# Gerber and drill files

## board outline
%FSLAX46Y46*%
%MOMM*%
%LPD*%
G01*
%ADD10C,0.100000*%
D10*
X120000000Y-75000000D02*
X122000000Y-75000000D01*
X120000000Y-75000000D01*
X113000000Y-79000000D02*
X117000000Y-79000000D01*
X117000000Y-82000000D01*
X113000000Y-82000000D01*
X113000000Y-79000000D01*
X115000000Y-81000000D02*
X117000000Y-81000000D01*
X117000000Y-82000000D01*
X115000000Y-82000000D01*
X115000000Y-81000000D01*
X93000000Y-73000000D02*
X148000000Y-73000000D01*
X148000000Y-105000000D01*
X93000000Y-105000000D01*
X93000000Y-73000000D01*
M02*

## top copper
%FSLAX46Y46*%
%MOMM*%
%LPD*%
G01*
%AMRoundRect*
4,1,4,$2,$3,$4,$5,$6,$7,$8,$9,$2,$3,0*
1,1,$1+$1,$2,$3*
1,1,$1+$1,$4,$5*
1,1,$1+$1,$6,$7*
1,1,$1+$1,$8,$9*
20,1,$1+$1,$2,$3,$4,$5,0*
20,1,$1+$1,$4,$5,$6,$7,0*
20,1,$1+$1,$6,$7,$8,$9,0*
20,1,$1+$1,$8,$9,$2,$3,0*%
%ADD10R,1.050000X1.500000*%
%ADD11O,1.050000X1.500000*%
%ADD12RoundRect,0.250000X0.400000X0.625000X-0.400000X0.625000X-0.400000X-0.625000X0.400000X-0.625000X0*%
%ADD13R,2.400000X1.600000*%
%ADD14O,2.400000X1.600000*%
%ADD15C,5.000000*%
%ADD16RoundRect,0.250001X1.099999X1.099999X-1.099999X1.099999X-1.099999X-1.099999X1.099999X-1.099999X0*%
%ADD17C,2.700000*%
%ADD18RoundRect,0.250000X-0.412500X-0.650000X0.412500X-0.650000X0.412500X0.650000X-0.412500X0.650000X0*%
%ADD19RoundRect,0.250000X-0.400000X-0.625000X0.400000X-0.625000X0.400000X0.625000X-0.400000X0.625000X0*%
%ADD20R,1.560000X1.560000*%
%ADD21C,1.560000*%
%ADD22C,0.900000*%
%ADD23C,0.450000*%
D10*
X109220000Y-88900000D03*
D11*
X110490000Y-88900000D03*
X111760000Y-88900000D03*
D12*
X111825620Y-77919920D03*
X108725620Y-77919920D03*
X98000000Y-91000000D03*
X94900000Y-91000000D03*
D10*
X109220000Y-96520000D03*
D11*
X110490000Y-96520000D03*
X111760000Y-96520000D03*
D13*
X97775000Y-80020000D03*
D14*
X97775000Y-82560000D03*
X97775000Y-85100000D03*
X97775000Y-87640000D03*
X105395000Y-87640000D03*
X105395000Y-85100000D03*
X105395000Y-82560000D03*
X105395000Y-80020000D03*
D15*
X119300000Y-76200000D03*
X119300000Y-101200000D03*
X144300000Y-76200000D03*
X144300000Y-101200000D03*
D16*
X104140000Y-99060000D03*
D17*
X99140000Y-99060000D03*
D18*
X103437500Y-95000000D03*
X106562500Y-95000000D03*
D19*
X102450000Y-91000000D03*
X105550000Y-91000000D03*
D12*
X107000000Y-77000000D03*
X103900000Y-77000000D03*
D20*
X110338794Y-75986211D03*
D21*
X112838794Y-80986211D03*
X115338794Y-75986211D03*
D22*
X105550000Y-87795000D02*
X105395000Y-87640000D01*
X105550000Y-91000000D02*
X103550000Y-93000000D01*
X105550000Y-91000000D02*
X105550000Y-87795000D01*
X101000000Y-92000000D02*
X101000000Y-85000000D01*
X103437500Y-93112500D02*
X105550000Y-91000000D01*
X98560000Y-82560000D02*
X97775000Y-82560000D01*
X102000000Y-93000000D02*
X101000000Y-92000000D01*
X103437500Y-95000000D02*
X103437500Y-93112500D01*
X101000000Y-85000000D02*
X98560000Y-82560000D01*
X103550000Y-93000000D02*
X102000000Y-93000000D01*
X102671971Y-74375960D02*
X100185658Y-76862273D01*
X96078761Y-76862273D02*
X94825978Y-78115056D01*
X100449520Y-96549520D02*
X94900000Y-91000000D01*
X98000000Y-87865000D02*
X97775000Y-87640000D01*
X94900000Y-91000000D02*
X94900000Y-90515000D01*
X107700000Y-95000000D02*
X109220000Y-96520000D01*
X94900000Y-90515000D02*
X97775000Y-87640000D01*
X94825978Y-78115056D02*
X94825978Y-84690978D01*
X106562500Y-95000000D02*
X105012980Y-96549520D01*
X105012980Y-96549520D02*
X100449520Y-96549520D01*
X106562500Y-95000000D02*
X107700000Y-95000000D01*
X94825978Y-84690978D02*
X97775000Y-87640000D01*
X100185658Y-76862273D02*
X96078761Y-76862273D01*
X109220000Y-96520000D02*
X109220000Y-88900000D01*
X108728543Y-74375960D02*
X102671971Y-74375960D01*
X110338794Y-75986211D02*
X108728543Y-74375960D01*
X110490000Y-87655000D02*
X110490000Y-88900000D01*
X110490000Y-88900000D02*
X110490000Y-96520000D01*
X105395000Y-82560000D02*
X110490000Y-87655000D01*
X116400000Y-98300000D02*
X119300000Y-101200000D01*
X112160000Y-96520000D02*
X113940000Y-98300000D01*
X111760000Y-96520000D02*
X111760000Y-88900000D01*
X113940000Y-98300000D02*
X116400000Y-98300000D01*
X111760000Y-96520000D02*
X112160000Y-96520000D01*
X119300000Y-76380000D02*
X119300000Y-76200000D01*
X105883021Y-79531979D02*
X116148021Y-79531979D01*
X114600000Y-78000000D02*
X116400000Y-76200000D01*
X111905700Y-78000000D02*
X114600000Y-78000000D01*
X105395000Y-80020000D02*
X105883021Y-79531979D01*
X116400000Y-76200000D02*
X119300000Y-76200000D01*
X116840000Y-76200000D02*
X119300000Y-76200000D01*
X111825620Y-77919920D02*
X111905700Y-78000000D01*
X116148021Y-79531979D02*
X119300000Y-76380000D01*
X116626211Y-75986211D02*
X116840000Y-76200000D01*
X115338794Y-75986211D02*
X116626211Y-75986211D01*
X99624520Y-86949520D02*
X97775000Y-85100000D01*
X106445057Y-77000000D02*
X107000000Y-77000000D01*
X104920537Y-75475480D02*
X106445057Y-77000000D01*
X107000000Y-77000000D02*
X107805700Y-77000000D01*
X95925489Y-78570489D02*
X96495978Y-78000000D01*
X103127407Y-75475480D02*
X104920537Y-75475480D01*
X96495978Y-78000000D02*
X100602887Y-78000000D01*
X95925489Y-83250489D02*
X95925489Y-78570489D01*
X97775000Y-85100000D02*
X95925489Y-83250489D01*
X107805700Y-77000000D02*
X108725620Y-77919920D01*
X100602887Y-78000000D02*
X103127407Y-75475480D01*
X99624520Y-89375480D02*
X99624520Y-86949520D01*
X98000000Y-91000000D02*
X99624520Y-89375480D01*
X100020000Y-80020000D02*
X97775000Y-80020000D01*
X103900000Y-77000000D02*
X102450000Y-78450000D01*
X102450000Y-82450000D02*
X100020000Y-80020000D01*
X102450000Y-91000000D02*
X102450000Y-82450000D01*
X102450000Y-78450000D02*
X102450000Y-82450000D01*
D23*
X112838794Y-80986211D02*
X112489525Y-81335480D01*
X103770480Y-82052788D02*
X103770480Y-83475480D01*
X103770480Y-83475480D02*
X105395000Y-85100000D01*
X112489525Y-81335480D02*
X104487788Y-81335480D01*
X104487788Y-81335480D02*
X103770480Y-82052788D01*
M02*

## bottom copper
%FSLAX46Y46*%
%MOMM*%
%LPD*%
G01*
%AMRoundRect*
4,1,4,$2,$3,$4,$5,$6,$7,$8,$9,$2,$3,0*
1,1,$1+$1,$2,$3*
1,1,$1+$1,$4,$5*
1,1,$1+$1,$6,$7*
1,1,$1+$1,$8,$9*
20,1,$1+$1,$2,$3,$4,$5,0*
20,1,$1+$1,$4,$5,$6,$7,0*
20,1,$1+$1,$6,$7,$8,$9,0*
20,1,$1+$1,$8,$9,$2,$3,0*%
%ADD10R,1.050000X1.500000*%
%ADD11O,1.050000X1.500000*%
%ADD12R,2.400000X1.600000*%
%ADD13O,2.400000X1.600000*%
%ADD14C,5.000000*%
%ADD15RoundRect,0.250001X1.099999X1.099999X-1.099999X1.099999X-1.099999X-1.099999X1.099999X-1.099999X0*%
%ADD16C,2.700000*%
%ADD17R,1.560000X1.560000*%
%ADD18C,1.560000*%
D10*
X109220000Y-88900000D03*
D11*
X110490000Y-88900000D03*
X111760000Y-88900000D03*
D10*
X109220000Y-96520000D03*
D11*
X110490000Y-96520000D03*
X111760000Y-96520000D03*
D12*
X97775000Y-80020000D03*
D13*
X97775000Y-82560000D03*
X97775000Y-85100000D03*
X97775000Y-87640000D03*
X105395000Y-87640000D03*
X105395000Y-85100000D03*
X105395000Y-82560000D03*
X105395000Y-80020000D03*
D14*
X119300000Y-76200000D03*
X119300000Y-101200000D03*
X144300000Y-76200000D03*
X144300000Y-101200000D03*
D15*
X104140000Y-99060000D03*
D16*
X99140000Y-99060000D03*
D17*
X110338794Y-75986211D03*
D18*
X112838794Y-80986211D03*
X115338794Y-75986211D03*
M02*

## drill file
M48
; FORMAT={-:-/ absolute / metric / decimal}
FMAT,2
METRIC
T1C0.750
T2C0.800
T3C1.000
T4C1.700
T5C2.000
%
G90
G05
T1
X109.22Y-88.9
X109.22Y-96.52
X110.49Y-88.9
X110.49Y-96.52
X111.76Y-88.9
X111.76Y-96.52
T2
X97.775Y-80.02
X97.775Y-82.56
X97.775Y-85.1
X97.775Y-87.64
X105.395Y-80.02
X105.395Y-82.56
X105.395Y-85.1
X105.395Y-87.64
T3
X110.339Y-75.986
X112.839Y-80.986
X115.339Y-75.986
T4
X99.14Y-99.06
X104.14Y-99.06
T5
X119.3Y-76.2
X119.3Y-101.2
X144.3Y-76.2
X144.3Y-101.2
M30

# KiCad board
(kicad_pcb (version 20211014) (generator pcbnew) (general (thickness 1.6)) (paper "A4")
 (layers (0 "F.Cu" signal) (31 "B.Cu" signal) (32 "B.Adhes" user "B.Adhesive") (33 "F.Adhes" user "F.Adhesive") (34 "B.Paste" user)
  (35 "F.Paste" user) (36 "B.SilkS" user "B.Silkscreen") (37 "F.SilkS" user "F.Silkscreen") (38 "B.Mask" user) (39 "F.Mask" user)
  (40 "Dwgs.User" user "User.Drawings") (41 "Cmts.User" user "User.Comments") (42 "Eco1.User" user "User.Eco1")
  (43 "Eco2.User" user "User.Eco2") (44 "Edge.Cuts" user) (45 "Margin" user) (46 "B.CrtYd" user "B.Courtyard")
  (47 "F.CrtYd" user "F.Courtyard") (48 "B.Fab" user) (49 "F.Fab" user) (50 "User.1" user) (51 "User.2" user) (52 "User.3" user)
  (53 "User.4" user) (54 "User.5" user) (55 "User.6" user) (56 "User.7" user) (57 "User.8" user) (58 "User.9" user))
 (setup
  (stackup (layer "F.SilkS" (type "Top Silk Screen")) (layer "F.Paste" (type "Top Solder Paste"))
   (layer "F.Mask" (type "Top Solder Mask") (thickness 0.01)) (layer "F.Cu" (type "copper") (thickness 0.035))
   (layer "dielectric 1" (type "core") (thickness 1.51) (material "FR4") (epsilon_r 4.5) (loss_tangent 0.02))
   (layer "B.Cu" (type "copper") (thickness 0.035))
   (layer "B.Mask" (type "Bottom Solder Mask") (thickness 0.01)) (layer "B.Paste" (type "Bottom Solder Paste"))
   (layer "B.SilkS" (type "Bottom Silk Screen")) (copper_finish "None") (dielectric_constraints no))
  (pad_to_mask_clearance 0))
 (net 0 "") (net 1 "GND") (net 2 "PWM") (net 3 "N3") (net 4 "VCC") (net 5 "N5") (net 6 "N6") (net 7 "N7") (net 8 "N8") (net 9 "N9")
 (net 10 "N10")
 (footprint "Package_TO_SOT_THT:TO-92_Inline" (layer "F.Cu") (at 109.22 88.9)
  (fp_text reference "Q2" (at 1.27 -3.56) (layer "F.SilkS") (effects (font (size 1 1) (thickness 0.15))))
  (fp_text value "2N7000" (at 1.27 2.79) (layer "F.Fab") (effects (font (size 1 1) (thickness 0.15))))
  (pad "1" thru_hole rect (at 0 0) (size 1.05 1.5) (drill 0.75) (layers *.Cu *.Mask) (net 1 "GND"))
  (pad "2" thru_hole oval (at 1.27 0) (size 1.05 1.5) (drill 0.75) (layers *.Cu *.Mask) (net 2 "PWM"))
  (pad "3" thru_hole oval (at 2.54 0) (size 1.05 1.5) (drill 0.75) (layers *.Cu *.Mask) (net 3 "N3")))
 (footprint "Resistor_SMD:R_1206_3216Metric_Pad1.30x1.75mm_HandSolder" (layer "F.Cu") (at 110.27562 77.91992 180)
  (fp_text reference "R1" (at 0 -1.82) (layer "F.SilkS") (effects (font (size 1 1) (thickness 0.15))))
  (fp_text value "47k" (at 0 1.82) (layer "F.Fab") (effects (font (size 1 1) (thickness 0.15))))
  (pad "1" smd roundrect (at -1.55 0 180) (size 1.3 1.75) (layers "F.Cu" "F.Paste" "F.Mask") (roundrect_rratio 0.192308) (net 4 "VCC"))
  (pad "2" smd roundrect (at 1.55 0 180) (size 1.3 1.75) (layers "F.Cu" "F.Paste" "F.Mask") (roundrect_rratio 0.192308) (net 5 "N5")))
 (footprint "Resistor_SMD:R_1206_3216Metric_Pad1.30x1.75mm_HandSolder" (layer "F.Cu") (at 96.45 91 180)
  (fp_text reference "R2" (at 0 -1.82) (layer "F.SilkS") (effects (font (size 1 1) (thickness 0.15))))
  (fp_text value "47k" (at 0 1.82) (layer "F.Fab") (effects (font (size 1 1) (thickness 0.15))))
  (pad "1" smd roundrect (at -1.55 0 180) (size 1.3 1.75) (layers "F.Cu" "F.Paste" "F.Mask") (roundrect_rratio 0.192308) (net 5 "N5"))
  (pad "2" smd roundrect (at 1.55 0 180) (size 1.3 1.75) (layers "F.Cu" "F.Paste" "F.Mask") (roundrect_rratio 0.192308) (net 1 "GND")))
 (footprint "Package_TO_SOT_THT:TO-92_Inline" (layer "F.Cu") (at 109.22 96.52)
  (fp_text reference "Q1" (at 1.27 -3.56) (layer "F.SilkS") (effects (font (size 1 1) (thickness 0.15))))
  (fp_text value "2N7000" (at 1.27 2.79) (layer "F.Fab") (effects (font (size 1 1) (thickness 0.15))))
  (pad "1" thru_hole rect (at 0 0) (size 1.05 1.5) (drill 0.75) (layers *.Cu *.Mask) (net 1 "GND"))
  (pad "2" thru_hole oval (at 1.27 0) (size 1.05 1.5) (drill 0.75) (layers *.Cu *.Mask) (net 2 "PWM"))
  (pad "3" thru_hole oval (at 2.54 0) (size 1.05 1.5) (drill 0.75) (layers *.Cu *.Mask) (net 3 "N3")))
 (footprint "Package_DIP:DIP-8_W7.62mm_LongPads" (layer "F.Cu") (at 97.775 80.02)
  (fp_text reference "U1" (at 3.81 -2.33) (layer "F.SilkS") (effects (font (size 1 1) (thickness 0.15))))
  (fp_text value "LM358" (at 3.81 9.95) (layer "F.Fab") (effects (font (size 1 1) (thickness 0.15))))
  (pad "1" thru_hole rect (at 0 0) (size 2.4 1.6) (drill 0.8) (layers *.Cu *.Mask) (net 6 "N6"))
  (pad "2" thru_hole oval (at 0 2.54) (size 2.4 1.6) (drill 0.8) (layers *.Cu *.Mask) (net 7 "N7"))
  (pad "3" thru_hole oval (at 0 5.08) (size 2.4 1.6) (drill 0.8) (layers *.Cu *.Mask) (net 5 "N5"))
  (pad "4" thru_hole oval (at 0 7.62) (size 2.4 1.6) (drill 0.8) (layers *.Cu *.Mask) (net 1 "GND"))
  (pad "5" thru_hole oval (at 7.62 7.62) (size 2.4 1.6) (drill 0.8) (layers *.Cu *.Mask) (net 7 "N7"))
  (pad "6" thru_hole oval (at 7.62 5.08) (size 2.4 1.6) (drill 0.8) (layers *.Cu *.Mask) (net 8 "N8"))
  (pad "7" thru_hole oval (at 7.62 2.54) (size 2.4 1.6) (drill 0.8) (layers *.Cu *.Mask) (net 2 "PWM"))
  (pad "8" thru_hole oval (at 7.62 0) (size 2.4 1.6) (drill 0.8) (layers *.Cu *.Mask) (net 4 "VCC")))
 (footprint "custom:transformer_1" (layer "F.Cu") (at 132 88.9)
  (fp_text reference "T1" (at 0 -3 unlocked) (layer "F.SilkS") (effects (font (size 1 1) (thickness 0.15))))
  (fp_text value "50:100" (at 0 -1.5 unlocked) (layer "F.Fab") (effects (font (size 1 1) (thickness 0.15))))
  (pad "1" thru_hole circle (at -12.7 -12.7) (size 5 5) (drill 2) (layers *.Cu *.Mask) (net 4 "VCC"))
  (pad "2" thru_hole circle (at -12.7 12.3) (size 5 5) (drill 2) (layers *.Cu *.Mask) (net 3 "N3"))
  (pad "3" thru_hole circle (at 12.3 -12.7) (size 5 5) (drill 2) (layers *.Cu *.Mask) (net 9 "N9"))
  (pad "4" thru_hole circle (at 12.3 12.3) (size 5 5) (drill 2) (layers *.Cu *.Mask) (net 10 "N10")))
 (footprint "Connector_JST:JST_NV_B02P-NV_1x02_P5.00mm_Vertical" (layer "F.Cu") (at 104.14 99.06 180)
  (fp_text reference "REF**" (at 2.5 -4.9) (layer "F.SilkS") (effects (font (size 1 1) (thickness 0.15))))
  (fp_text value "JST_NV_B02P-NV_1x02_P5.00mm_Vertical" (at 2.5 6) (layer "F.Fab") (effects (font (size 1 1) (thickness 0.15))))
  (pad "1" thru_hole roundrect (at 0 0 180) (size 2.7 2.7) (drill 1.7) (layers *.Cu *.Mask) (roundrect_rratio 0.092593))
  (pad "2" thru_hole circle (at 5 0 180) (size 2.7 2.7) (drill 1.7) (layers *.Cu *.Mask)))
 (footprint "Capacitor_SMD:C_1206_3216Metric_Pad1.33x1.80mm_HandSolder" (layer "F.Cu") (at 105 95)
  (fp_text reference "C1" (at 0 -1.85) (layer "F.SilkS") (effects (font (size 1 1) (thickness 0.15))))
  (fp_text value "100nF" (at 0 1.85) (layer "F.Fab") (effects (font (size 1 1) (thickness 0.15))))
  (pad "1" smd roundrect (at -1.5625 0) (size 1.325 1.8) (layers "F.Cu" "F.Paste" "F.Mask") (roundrect_rratio 0.188679) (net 7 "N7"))
  (pad "2" smd roundrect (at 1.5625 0) (size 1.325 1.8) (layers "F.Cu" "F.Paste" "F.Mask") (roundrect_rratio 0.188679) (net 1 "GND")))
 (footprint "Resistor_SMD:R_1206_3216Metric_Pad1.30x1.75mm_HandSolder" (layer "F.Cu") (at 104 91)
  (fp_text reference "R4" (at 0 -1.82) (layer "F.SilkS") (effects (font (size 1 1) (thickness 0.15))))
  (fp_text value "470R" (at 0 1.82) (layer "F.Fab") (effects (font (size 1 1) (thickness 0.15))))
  (pad "1" smd roundrect (at -1.55 0) (size 1.3 1.75) (layers "F.Cu" "F.Paste" "F.Mask") (roundrect_rratio 0.192308) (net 6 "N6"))
  (pad "2" smd roundrect (at 1.55 0) (size 1.3 1.75) (layers "F.Cu" "F.Paste" "F.Mask") (roundrect_rratio 0.192308) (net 7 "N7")))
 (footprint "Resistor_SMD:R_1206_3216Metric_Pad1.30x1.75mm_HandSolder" (layer "F.Cu") (at 105.45 77 180)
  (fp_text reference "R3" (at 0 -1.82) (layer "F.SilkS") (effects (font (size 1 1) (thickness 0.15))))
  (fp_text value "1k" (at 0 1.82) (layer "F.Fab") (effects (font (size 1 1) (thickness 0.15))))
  (pad "1" smd roundrect (at -1.55 0 180) (size 1.3 1.75) (layers "F.Cu" "F.Paste" "F.Mask") (roundrect_rratio 0.192308) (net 5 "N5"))
  (pad "2" smd roundrect (at 1.55 0 180) (size 1.3 1.75) (layers "F.Cu" "F.Paste" "F.Mask") (roundrect_rratio 0.192308) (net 6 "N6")))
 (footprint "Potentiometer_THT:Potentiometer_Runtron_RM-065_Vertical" (layer "F.Cu") (at 110.338794 75.986211)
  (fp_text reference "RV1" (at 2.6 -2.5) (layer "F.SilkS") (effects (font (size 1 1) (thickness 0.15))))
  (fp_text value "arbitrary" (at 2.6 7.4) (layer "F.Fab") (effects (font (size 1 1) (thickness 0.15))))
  (pad "1" thru_hole rect (at 0 0) (size 1.56 1.56) (drill 1) (layers *.Cu *.Mask) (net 1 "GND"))
  (pad "2" thru_hole circle (at 2.5 5) (size 1.56 1.56) (drill 1) (layers *.Cu *.Mask) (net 8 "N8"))
  (pad "3" thru_hole circle (at 5 0) (size 1.56 1.56) (drill 1) (layers *.Cu *.Mask) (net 4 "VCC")))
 (gr_rect (start 122 75) (end 120 75) (layer "Edge.Cuts") (width 0.1) (fill none))
 (gr_rect (start 113 79) (end 117 82) (layer "Edge.Cuts") (width 0.1) (fill none))
 (gr_rect (start 117 82) (end 115 81) (layer "Edge.Cuts") (width 0.1) (fill none))
 (gr_rect (start 93 73) (end 148 105) (layer "Edge.Cuts") (width 0.1) (fill none))
 (segment (start 105.55 87.795) (end 105.395 87.64) (width 0.9) (layer "F.Cu") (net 7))
 (segment (start 105.55 91) (end 103.55 93) (width 0.9) (layer "F.Cu") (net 7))
 (segment (start 105.55 91) (end 105.55 87.795) (width 0.9) (layer "F.Cu") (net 7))
 (segment (start 101 92) (end 101 85) (width 0.9) (layer "F.Cu") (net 7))
 (segment (start 103.4375 93.1125) (end 105.55 91) (width 0.9) (layer "F.Cu") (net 7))
 (segment (start 98.56 82.56) (end 97.775 82.56) (width 0.9) (layer "F.Cu") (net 7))
 (segment (start 102 93) (end 101 92) (width 0.9) (layer "F.Cu") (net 7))
 (segment (start 103.4375 95) (end 103.4375 93.1125) (width 0.9) (layer "F.Cu") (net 7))
 (segment (start 101 85) (end 98.56 82.56) (width 0.9) (layer "F.Cu") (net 7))
 (segment (start 103.55 93) (end 102 93) (width 0.9) (layer "F.Cu") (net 7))
 (segment (start 102.671971 74.37596) (end 100.185658 76.862273) (width 0.9) (layer "F.Cu") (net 1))
 (segment (start 96.078761 76.862273) (end 94.825978 78.115056) (width 0.9) (layer "F.Cu") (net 1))
 (segment (start 100.44952 96.54952) (end 94.9 91) (width 0.9) (layer "F.Cu") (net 1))
 (segment (start 98 87.865) (end 97.775 87.64) (width 0.9) (layer "F.Cu") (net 1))
 (segment (start 94.9 91) (end 94.9 90.515) (width 0.9) (layer "F.Cu") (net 1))
 (segment (start 107.7 95) (end 109.22 96.52) (width 0.9) (layer "F.Cu") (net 1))
 (segment (start 94.9 90.515) (end 97.775 87.64) (width 0.9) (layer "F.Cu") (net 1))
 (segment (start 94.825978 78.115056) (end 94.825978 84.690978) (width 0.9) (layer "F.Cu") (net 1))
 (segment (start 106.5625 95) (end 105.01298 96.54952) (width 0.9) (layer "F.Cu") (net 1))
 (segment (start 105.01298 96.54952) (end 100.44952 96.54952) (width 0.9) (layer "F.Cu") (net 1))
 (segment (start 106.5625 95) (end 107.7 95) (width 0.9) (layer "F.Cu") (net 1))
 (segment (start 94.825978 84.690978) (end 97.775 87.64) (width 0.9) (layer "F.Cu") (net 1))
 (segment (start 100.185658 76.862273) (end 96.078761 76.862273) (width 0.9) (layer "F.Cu") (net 1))
 (segment (start 109.22 96.52) (end 109.22 88.9) (width 0.9) (layer "F.Cu") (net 1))
 (segment (start 108.728543 74.37596) (end 102.671971 74.37596) (width 0.9) (layer "F.Cu") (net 1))
 (segment (start 110.338794 75.986211) (end 108.728543 74.37596) (width 0.9) (layer "F.Cu") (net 1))
 (segment (start 110.49 87.655) (end 110.49 88.9) (width 0.9) (layer "F.Cu") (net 2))
 (segment (start 110.49 88.9) (end 110.49 96.52) (width 0.9) (layer "F.Cu") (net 2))
 (segment (start 105.395 82.56) (end 110.49 87.655) (width 0.9) (layer "F.Cu") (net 2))
 (segment (start 116.4 98.3) (end 119.3 101.2) (width 0.9) (layer "F.Cu") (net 3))
 (segment (start 112.16 96.52) (end 113.94 98.3) (width 0.9) (layer "F.Cu") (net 3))
 (segment (start 111.76 96.52) (end 111.76 88.9) (width 0.9) (layer "F.Cu") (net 3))
 (segment (start 113.94 98.3) (end 116.4 98.3) (width 0.9) (layer "F.Cu") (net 3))
 (segment (start 111.76 96.52) (end 112.16 96.52) (width 0.9) (layer "F.Cu") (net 3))
 (segment (start 119.3 76.38) (end 119.3 76.2) (width 0.9) (layer "F.Cu") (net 4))
 (segment (start 105.883021 79.531979) (end 116.148021 79.531979) (width 0.9) (layer "F.Cu") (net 4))
 (segment (start 114.6 78) (end 116.4 76.2) (width 0.9) (layer "F.Cu") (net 4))
 (segment (start 111.9057 78) (end 114.6 78) (width 0.9) (layer "F.Cu") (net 4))
 (segment (start 105.395 80.02) (end 105.883021 79.531979) (width 0.9) (layer "F.Cu") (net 4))
 (segment (start 116.4 76.2) (end 119.3 76.2) (width 0.9) (layer "F.Cu") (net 4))
 (segment (start 116.84 76.2) (end 119.3 76.2) (width 0.9) (layer "F.Cu") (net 4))
 (segment (start 111.82562 77.91992) (end 111.9057 78) (width 0.9) (layer "F.Cu") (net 4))
 (segment (start 116.148021 79.531979) (end 119.3 76.38) (width 0.9) (layer "F.Cu") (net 4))
 (segment (start 116.626211 75.986211) (end 116.84 76.2) (width 0.9) (layer "F.Cu") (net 4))
 (segment (start 115.338794 75.986211) (end 116.626211 75.986211) (width 0.9) (layer "F.Cu") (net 4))
 (segment (start 99.62452 86.94952) (end 97.775 85.1) (width 0.9) (layer "F.Cu") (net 5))
 (segment (start 106.445057 77) (end 107 77) (width 0.9) (layer "F.Cu") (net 5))
 (segment (start 104.920537 75.47548) (end 106.445057 77) (width 0.9) (layer "F.Cu") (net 5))
 (segment (start 107 77) (end 107.8057 77) (width 0.9) (layer "F.Cu") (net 5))
 (segment (start 95.925489 78.570489) (end 96.495978 78) (width 0.9) (layer "F.Cu") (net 5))
 (segment (start 103.127407 75.47548) (end 104.920537 75.47548) (width 0.9) (layer "F.Cu") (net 5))
 (segment (start 96.495978 78) (end 100.602887 78) (width 0.9) (layer "F.Cu") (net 5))
 (segment (start 95.925489 83.250489) (end 95.925489 78.570489) (width 0.9) (layer "F.Cu") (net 5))
 (segment (start 97.775 85.1) (end 95.925489 83.250489) (width 0.9) (layer "F.Cu") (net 5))
 (segment (start 107.8057 77) (end 108.72562 77.91992) (width 0.9) (layer "F.Cu") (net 5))
 (segment (start 100.602887 78) (end 103.127407 75.47548) (width 0.9) (layer "F.Cu") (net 5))
 (segment (start 99.62452 89.37548) (end 99.62452 86.94952) (width 0.9) (layer "F.Cu") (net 5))
 (segment (start 98 91) (end 99.62452 89.37548) (width 0.9) (layer "F.Cu") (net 5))
 (segment (start 100.02 80.02) (end 97.775 80.02) (width 0.9) (layer "F.Cu") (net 6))
 (segment (start 103.9 77) (end 102.45 78.45) (width 0.9) (layer "F.Cu") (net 6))
 (segment (start 102.45 82.45) (end 100.02 80.02) (width 0.9) (layer "F.Cu") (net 6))
 (segment (start 102.45 91) (end 102.45 82.45) (width 0.9) (layer "F.Cu") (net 6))
 (segment (start 102.45 78.45) (end 102.45 82.45) (width 0.9) (layer "F.Cu") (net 6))
 (segment (start 112.838794 80.986211) (end 112.489525 81.33548) (width 0.45) (layer "F.Cu") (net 8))
 (segment (start 103.77048 82.052788) (end 103.77048 83.47548) (width 0.45) (layer "F.Cu") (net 8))
 (segment (start 103.77048 83.47548) (end 105.395 85.1) (width 0.45) (layer "F.Cu") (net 8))
 (segment (start 112.489525 81.33548) (end 104.487788 81.33548) (width 0.45) (layer "F.Cu") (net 8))
 (segment (start 104.487788 81.33548) (end 103.77048 82.052788) (width 0.45) (layer "F.Cu") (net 8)))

